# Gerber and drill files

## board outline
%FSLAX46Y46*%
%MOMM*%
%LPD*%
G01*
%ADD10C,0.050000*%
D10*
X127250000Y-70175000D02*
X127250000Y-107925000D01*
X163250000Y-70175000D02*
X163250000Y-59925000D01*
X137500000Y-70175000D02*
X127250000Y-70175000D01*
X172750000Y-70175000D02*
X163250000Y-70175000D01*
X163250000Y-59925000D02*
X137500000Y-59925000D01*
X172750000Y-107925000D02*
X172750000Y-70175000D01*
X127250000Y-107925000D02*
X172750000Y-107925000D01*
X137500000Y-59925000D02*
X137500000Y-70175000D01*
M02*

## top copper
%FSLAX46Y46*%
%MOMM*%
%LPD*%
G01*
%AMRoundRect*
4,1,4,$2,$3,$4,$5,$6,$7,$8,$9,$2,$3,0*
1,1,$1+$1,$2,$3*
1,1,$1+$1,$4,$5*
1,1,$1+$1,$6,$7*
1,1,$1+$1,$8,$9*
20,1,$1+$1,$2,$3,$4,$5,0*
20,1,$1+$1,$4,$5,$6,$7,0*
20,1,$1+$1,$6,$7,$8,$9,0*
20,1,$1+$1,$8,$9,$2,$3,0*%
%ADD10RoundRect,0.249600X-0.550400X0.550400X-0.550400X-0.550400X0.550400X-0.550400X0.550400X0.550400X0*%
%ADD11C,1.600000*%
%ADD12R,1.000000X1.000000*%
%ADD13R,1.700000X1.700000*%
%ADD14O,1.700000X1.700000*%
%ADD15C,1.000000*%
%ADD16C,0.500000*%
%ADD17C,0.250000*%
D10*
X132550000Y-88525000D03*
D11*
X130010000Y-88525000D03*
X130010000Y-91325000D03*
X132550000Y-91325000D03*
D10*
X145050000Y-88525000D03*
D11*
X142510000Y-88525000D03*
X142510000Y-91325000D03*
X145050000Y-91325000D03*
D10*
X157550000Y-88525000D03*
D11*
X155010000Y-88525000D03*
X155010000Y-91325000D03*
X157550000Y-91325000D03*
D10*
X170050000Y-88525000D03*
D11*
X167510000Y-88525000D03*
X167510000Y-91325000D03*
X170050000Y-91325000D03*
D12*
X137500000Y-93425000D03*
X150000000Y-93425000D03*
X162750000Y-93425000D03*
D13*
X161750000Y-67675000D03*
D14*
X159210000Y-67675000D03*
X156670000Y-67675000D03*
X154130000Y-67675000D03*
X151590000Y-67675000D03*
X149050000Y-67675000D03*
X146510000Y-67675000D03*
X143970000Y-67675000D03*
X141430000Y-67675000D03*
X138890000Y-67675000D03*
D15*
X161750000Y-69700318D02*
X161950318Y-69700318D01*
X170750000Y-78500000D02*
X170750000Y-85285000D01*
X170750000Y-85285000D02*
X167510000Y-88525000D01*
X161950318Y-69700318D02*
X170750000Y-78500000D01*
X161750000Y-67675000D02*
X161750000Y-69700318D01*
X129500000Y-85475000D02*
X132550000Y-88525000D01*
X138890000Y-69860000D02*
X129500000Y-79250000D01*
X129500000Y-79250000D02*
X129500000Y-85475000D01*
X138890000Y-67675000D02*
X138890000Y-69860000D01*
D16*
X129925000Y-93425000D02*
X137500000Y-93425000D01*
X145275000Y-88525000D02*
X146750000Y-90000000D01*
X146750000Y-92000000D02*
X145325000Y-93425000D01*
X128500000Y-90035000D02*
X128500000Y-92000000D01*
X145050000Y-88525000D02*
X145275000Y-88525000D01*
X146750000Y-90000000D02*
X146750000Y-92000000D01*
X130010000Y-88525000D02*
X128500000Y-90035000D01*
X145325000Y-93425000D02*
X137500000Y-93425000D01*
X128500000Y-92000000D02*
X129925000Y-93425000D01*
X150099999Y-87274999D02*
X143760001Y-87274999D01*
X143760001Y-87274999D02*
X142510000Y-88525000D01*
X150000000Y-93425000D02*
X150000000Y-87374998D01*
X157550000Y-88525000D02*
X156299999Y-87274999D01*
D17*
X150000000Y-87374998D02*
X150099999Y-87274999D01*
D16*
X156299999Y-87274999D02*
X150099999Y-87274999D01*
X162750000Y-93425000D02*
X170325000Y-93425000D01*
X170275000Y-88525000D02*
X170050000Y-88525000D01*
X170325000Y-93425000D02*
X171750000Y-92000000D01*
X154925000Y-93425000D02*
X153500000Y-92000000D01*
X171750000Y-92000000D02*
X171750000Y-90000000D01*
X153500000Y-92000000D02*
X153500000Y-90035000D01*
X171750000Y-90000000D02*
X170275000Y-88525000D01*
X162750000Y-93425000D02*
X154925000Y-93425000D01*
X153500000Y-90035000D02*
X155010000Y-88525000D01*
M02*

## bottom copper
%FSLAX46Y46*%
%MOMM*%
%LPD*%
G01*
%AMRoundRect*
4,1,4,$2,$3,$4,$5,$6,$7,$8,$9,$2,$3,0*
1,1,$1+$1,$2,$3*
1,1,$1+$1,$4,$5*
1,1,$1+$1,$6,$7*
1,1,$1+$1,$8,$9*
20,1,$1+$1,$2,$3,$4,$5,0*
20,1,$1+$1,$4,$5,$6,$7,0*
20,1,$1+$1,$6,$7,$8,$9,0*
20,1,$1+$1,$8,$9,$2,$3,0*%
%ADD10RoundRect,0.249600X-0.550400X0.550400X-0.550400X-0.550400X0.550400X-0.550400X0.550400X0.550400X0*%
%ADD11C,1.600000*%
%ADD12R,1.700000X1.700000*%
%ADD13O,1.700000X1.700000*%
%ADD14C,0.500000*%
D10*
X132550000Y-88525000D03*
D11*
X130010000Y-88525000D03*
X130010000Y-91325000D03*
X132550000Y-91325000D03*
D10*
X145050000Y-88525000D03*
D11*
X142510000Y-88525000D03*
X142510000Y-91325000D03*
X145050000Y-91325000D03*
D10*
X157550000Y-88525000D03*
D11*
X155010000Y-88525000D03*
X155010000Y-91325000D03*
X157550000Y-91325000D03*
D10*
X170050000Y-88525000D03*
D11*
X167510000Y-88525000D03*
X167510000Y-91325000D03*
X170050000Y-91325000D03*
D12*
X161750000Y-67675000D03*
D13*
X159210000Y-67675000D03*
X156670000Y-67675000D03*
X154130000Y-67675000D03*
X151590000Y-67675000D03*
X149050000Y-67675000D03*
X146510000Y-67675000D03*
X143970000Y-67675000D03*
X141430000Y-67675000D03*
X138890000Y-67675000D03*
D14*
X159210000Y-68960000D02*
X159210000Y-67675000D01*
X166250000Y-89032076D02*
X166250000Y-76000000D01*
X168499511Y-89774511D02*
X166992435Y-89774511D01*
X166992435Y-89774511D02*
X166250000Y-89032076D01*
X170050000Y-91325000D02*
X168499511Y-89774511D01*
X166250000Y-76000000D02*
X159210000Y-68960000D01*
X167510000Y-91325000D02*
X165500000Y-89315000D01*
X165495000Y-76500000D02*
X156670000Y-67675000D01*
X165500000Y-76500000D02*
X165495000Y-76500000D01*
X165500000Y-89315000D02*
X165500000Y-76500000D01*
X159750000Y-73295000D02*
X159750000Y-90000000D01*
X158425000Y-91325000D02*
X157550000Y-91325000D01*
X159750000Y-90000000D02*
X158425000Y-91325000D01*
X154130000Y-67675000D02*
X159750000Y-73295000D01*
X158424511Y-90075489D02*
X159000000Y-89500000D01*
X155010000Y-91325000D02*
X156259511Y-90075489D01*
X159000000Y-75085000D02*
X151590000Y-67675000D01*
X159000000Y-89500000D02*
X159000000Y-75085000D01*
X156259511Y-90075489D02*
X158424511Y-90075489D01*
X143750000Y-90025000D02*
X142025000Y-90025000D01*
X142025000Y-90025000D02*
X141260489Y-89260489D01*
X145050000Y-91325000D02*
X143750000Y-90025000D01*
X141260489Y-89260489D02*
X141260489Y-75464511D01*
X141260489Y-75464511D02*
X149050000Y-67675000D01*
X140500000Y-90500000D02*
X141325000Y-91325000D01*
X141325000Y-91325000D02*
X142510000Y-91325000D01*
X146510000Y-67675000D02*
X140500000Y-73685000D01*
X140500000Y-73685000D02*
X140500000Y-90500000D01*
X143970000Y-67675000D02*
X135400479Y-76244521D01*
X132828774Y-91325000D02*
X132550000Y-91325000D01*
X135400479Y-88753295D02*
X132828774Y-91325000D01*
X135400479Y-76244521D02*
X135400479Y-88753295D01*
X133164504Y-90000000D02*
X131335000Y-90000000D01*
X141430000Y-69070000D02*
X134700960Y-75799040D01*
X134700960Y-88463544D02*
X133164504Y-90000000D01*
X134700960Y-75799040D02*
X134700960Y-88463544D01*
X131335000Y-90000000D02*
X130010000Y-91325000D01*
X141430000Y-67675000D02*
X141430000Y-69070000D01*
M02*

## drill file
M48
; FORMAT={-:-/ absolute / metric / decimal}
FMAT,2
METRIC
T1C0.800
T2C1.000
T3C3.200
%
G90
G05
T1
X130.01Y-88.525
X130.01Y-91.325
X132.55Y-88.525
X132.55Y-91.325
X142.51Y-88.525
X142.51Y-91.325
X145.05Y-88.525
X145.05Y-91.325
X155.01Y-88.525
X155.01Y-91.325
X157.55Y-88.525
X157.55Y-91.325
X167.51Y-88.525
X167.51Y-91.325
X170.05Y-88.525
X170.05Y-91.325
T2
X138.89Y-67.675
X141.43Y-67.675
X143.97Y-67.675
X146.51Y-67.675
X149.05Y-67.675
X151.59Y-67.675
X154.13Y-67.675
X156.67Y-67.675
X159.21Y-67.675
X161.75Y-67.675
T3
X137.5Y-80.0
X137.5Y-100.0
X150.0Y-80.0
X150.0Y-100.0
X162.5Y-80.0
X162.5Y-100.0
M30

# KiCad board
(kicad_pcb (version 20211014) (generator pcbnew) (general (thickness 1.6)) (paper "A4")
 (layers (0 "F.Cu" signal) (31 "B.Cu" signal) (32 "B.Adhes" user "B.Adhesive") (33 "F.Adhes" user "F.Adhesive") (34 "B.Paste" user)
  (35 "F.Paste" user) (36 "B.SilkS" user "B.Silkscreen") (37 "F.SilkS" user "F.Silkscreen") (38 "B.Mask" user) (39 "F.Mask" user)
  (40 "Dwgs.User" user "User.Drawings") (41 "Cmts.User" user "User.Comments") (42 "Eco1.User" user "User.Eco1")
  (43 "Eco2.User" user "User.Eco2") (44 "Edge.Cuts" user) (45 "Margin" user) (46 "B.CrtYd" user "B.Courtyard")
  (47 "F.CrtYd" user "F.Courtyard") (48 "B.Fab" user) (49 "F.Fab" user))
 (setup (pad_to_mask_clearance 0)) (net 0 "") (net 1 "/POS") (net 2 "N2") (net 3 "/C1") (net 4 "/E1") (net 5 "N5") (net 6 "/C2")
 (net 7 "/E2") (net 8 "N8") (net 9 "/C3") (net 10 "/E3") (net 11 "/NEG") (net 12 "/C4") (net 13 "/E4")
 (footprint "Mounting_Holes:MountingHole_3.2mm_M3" (layer "F.Cu") (at 137.5 100)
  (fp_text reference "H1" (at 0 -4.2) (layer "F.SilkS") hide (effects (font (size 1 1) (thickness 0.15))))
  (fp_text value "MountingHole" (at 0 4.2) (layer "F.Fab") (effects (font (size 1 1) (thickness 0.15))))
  (pad "" np_thru_hole circle locked (at 0 0) (size 3.2 3.2) (drill 3.2) (layers *.Cu *.Mask)))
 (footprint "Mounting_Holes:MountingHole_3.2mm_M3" (layer "F.Cu") (at 137.5 80)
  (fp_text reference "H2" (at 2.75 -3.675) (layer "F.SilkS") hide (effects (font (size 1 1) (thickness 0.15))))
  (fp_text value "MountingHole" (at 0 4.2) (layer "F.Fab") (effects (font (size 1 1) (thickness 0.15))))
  (pad "" np_thru_hole circle locked (at 0 0) (size 3.2 3.2) (drill 3.2) (layers *.Cu *.Mask)))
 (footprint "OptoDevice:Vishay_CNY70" (layer "F.Cu") (at 132.55 88.525 -90)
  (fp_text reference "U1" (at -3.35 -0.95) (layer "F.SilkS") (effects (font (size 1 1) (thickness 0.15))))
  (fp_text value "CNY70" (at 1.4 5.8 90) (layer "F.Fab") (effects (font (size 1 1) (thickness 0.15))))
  (pad "1" thru_hole roundrect (at 0 0 270) (size 1.6 1.6) (drill 0.8) (layers *.Cu *.Mask) (roundrect_rratio 0.156) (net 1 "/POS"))
  (pad "2" thru_hole circle (at 0 2.54 270) (size 1.6 1.6) (drill 0.8) (layers *.Cu *.Mask) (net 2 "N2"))
  (pad "3" thru_hole circle (at 2.8 2.54 270) (size 1.6 1.6) (drill 0.8) (layers *.Cu *.Mask) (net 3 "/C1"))
  (pad "4" thru_hole circle (at 2.8 0 270) (size 1.6 1.6) (drill 0.8) (layers *.Cu *.Mask) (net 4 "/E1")))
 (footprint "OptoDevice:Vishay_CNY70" (layer "F.Cu") (at 145.05 88.525 -90)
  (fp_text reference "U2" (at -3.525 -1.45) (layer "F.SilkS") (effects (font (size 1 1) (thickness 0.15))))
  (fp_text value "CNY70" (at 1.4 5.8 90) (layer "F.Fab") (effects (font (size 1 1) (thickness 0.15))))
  (pad "1" thru_hole roundrect (at 0 0 270) (size 1.6 1.6) (drill 0.8) (layers *.Cu *.Mask) (roundrect_rratio 0.156) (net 2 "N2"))
  (pad "2" thru_hole circle (at 0 2.54 270) (size 1.6 1.6) (drill 0.8) (layers *.Cu *.Mask) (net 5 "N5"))
  (pad "3" thru_hole circle (at 2.8 2.54 270) (size 1.6 1.6) (drill 0.8) (layers *.Cu *.Mask) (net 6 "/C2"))
  (pad "4" thru_hole circle (at 2.8 0 270) (size 1.6 1.6) (drill 0.8) (layers *.Cu *.Mask) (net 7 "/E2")))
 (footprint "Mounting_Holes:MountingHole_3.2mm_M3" (layer "F.Cu") (at 150 100)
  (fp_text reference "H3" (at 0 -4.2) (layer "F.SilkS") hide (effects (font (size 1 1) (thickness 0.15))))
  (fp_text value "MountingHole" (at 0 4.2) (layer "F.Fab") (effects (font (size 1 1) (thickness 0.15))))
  (pad "" np_thru_hole circle locked (at 0 0) (size 3.2 3.2) (drill 3.2) (layers *.Cu *.Mask)))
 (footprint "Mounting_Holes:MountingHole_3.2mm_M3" (layer "F.Cu") (at 150 80)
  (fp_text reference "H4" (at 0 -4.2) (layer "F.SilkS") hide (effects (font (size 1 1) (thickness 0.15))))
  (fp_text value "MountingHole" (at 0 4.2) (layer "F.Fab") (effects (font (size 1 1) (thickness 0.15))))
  (pad "" np_thru_hole circle locked (at 0 0) (size 3.2 3.2) (drill 3.2) (layers *.Cu *.Mask)))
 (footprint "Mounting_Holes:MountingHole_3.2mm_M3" (layer "F.Cu") (at 162.5 100)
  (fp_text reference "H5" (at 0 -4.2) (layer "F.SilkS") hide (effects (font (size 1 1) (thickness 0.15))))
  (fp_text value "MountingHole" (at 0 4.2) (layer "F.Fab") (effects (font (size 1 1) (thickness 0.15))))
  (pad "" np_thru_hole circle locked (at 0 0) (size 3.2 3.2) (drill 3.2) (layers *.Cu *.Mask)))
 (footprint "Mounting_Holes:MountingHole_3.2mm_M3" (layer "F.Cu") (at 162.5 80)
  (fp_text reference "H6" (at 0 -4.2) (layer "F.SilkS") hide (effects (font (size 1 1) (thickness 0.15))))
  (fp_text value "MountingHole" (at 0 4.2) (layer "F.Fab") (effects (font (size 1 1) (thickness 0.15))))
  (pad "" np_thru_hole circle locked (at 0 0) (size 3.2 3.2) (drill 3.2) (layers *.Cu *.Mask)))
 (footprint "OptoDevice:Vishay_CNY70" (layer "F.Cu") (at 157.55 88.525 -90)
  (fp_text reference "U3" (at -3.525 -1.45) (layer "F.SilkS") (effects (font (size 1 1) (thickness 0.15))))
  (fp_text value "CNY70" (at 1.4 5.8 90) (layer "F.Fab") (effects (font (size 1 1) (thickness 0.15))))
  (pad "1" thru_hole roundrect (at 0 0 270) (size 1.6 1.6) (drill 0.8) (layers *.Cu *.Mask) (roundrect_rratio 0.156) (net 5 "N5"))
  (pad "2" thru_hole circle (at 0 2.54 270) (size 1.6 1.6) (drill 0.8) (layers *.Cu *.Mask) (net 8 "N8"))
  (pad "3" thru_hole circle (at 2.8 2.54 270) (size 1.6 1.6) (drill 0.8) (layers *.Cu *.Mask) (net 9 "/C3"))
  (pad "4" thru_hole circle (at 2.8 0 270) (size 1.6 1.6) (drill 0.8) (layers *.Cu *.Mask) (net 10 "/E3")))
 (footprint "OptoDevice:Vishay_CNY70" (layer "F.Cu") (at 170.05 88.525 -90)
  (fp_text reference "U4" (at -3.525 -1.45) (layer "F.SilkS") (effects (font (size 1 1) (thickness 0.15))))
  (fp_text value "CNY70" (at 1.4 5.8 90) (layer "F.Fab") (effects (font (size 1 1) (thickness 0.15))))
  (pad "1" thru_hole roundrect (at 0 0 270) (size 1.6 1.6) (drill 0.8) (layers *.Cu *.Mask) (roundrect_rratio 0.156) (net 8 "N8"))
  (pad "2" thru_hole circle (at 0 2.54 270) (size 1.6 1.6) (drill 0.8) (layers *.Cu *.Mask) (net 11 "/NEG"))
  (pad "3" thru_hole circle (at 2.8 2.54 270) (size 1.6 1.6) (drill 0.8) (layers *.Cu *.Mask) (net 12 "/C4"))
  (pad "4" thru_hole circle (at 2.8 0 270) (size 1.6 1.6) (drill 0.8) (layers *.Cu *.Mask) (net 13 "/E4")))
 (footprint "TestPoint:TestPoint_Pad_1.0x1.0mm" (layer "F.Cu") (at 137.5 93.425)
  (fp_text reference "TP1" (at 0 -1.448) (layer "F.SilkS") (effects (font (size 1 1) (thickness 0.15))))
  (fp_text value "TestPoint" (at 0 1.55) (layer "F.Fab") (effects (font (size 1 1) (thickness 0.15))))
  (pad "1" smd rect locked (at 0 0) (size 1 1) (layers "F.Cu" "F.Mask") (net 2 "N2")))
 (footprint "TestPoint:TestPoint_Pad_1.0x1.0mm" (layer "F.Cu") (at 150 93.425)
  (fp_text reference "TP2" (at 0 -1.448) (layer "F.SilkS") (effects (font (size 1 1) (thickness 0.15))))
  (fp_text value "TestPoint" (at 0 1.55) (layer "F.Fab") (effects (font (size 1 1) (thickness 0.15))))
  (pad "1" smd rect locked (at 0 0) (size 1 1) (layers "F.Cu" "F.Mask") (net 5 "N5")))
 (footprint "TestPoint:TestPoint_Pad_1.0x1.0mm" (layer "F.Cu") (at 162.75 93.425)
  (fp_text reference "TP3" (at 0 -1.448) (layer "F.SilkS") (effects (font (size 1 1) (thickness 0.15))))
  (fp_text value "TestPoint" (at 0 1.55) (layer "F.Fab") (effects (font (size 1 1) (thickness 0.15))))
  (pad "1" smd rect locked (at 0 0) (size 1 1) (layers "F.Cu" "F.Mask") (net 8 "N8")))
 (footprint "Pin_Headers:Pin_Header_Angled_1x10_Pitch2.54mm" (layer "B.Cu") (at 161.75 67.675 90)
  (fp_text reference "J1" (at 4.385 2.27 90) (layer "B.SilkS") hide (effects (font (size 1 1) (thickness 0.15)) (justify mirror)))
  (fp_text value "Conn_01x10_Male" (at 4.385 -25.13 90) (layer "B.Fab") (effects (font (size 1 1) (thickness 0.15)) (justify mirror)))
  (pad "1" thru_hole rect (at 0 0 90) (size 1.7 1.7) (drill 1) (layers *.Cu *.Mask) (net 11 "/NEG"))
  (pad "2" thru_hole oval (at 0 -2.54 90) (size 1.7 1.7) (drill 1) (layers *.Cu *.Mask) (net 13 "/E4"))
  (pad "3" thru_hole oval (at 0 -5.08 90) (size 1.7 1.7) (drill 1) (layers *.Cu *.Mask) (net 12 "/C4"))
  (pad "4" thru_hole oval (at 0 -7.62 90) (size 1.7 1.7) (drill 1) (layers *.Cu *.Mask) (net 10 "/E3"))
  (pad "5" thru_hole oval (at 0 -10.16 90) (size 1.7 1.7) (drill 1) (layers *.Cu *.Mask) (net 9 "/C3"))
  (pad "6" thru_hole oval (at 0 -12.7 90) (size 1.7 1.7) (drill 1) (layers *.Cu *.Mask) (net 7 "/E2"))
  (pad "7" thru_hole oval (at 0 -15.24 90) (size 1.7 1.7) (drill 1) (layers *.Cu *.Mask) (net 6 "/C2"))
  (pad "8" thru_hole oval (at 0 -17.78 90) (size 1.7 1.7) (drill 1) (layers *.Cu *.Mask) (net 4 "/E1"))
  (pad "9" thru_hole oval (at 0 -20.32 90) (size 1.7 1.7) (drill 1) (layers *.Cu *.Mask) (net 3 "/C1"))
  (pad "10" thru_hole oval (at 0 -22.86 90) (size 1.7 1.7) (drill 1) (layers *.Cu *.Mask) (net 1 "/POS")))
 (gr_line (start 127.25 70.175) (end 127.25 107.925) (layer "Edge.Cuts") (width 0.05))
 (gr_line (start 163.25 70.175) (end 163.25 59.925) (layer "Edge.Cuts") (width 0.05))
 (gr_line (start 137.5 70.175) (end 127.25 70.175) (layer "Edge.Cuts") (width 0.05))
 (gr_line (start 172.75 70.175) (end 163.25 70.175) (layer "Edge.Cuts") (width 0.05))
 (gr_line (start 163.25 59.925) (end 137.5 59.925) (layer "Edge.Cuts") (width 0.05))
 (gr_line (start 172.75 107.925) (end 172.75 70.175) (layer "Edge.Cuts") (width 0.05))
 (gr_line (start 127.25 107.925) (end 172.75 107.925) (layer "Edge.Cuts") (width 0.05))
 (gr_line (start 137.5 59.925) (end 137.5 70.175) (layer "Edge.Cuts") (width 0.05))
 (segment (start 161.75 69.700318) (end 161.950318 69.700318) (width 1) (layer "F.Cu") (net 11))
 (segment (start 170.75 78.5) (end 170.75 85.285) (width 1) (layer "F.Cu") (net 11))
 (segment (start 170.75 85.285) (end 167.51 88.525) (width 1) (layer "F.Cu") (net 11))
 (segment (start 161.950318 69.700318) (end 170.75 78.5) (width 1) (layer "F.Cu") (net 11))
 (segment (start 161.75 67.675) (end 161.75 69.700318) (width 1) (layer "F.Cu") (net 11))
 (segment (start 129.5 85.475) (end 132.55 88.525) (width 1) (layer "F.Cu") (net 1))
 (segment (start 138.89 69.86) (end 129.5 79.25) (width 1) (layer "F.Cu") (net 1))
 (segment (start 129.5 79.25) (end 129.5 85.475) (width 1) (layer "F.Cu") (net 1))
 (segment (start 138.89 67.675) (end 138.89 69.86) (width 1) (layer "F.Cu") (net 1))
 (segment (start 159.21 68.96) (end 159.21 67.675) (width 0.5) (layer "B.Cu") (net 13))
 (segment (start 166.25 89.032076) (end 166.25 76) (width 0.5) (layer "B.Cu") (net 13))
 (segment (start 168.499511 89.774511) (end 166.992435 89.774511) (width 0.5) (layer "B.Cu") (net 13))
 (segment (start 166.992435 89.774511) (end 166.25 89.032076) (width 0.5) (layer "B.Cu") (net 13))
 (segment (start 170.05 91.325) (end 168.499511 89.774511) (width 0.5) (layer "B.Cu") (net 13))
 (segment (start 166.25 76) (end 159.21 68.96) (width 0.5) (layer "B.Cu") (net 13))
 (segment (start 167.51 91.325) (end 165.5 89.315) (width 0.5) (layer "B.Cu") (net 12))
 (segment (start 165.495 76.5) (end 156.67 67.675) (width 0.5) (layer "B.Cu") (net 12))
 (segment (start 165.5 76.5) (end 165.495 76.5) (width 0.5) (layer "B.Cu") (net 12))
 (segment (start 165.5 89.315) (end 165.5 76.5) (width 0.5) (layer "B.Cu") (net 12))
 (segment (start 159.75 73.295) (end 159.75 90) (width 0.5) (layer "B.Cu") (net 10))
 (segment (start 158.425 91.325) (end 157.55 91.325) (width 0.5) (layer "B.Cu") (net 10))
 (segment (start 159.75 90) (end 158.425 91.325) (width 0.5) (layer "B.Cu") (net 10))
 (segment (start 154.13 67.675) (end 159.75 73.295) (width 0.5) (layer "B.Cu") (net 10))
 (segment (start 158.424511 90.075489) (end 159 89.5) (width 0.5) (layer "B.Cu") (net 9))
 (segment (start 155.01 91.325) (end 156.259511 90.075489) (width 0.5) (layer "B.Cu") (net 9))
 (segment (start 159 75.085) (end 151.59 67.675) (width 0.5) (layer "B.Cu") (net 9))
 (segment (start 159 89.5) (end 159 75.085) (width 0.5) (layer "B.Cu") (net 9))
 (segment (start 156.259511 90.075489) (end 158.424511 90.075489) (width 0.5) (layer "B.Cu") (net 9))
 (segment (start 143.75 90.025) (end 142.025 90.025) (width 0.5) (layer "B.Cu") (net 7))
 (segment (start 142.025 90.025) (end 141.260489 89.260489) (width 0.5) (layer "B.Cu") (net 7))
 (segment (start 145.05 91.325) (end 143.75 90.025) (width 0.5) (layer "B.Cu") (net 7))
 (segment (start 141.260489 89.260489) (end 141.260489 75.464511) (width 0.5) (layer "B.Cu") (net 7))
 (segment (start 141.260489 75.464511) (end 149.05 67.675) (width 0.5) (layer "B.Cu") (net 7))
 (segment (start 140.5 90.5) (end 141.325 91.325) (width 0.5) (layer "B.Cu") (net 6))
 (segment (start 141.325 91.325) (end 142.51 91.325) (width 0.5) (layer "B.Cu") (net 6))
 (segment (start 146.51 67.675) (end 140.5 73.685) (width 0.5) (layer "B.Cu") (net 6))
 (segment (start 140.5 73.685) (end 140.5 90.5) (width 0.5) (layer "B.Cu") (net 6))
 (segment (start 143.97 67.675) (end 135.400479 76.244521) (width 0.5) (layer "B.Cu") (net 4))
 (segment (start 132.828774 91.325) (end 132.55 91.325) (width 0.5) (layer "B.Cu") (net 4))
 (segment (start 135.400479 88.753295) (end 132.828774 91.325) (width 0.5) (layer "B.Cu") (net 4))
 (segment (start 135.400479 76.244521) (end 135.400479 88.753295) (width 0.5) (layer "B.Cu") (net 4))
 (segment (start 133.164504 90) (end 131.335 90) (width 0.5) (layer "B.Cu") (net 3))
 (segment (start 141.43 69.07) (end 134.70096 75.79904) (width 0.5) (layer "B.Cu") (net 3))
 (segment (start 134.70096 88.463544) (end 133.164504 90) (width 0.5) (layer "B.Cu") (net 3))
 (segment (start 134.70096 75.79904) (end 134.70096 88.463544) (width 0.5) (layer "B.Cu") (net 3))
 (segment (start 131.335 90) (end 130.01 91.325) (width 0.5) (layer "B.Cu") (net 3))
 (segment (start 141.43 67.675) (end 141.43 69.07) (width 0.5) (layer "B.Cu") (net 3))
 (segment (start 129.925 93.425) (end 137.5 93.425) (width 0.5) (layer "F.Cu") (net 2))
 (segment (start 145.275 88.525) (end 146.75 90) (width 0.5) (layer "F.Cu") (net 2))
 (segment (start 146.75 92) (end 145.325 93.425) (width 0.5) (layer "F.Cu") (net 2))
 (segment (start 128.5 90.035) (end 128.5 92) (width 0.5) (layer "F.Cu") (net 2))
 (segment (start 145.05 88.525) (end 145.275 88.525) (width 0.5) (layer "F.Cu") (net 2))
 (segment (start 146.75 90) (end 146.75 92) (width 0.5) (layer "F.Cu") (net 2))
 (segment (start 130.01 88.525) (end 128.5 90.035) (width 0.5) (layer "F.Cu") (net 2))
 (segment (start 145.325 93.425) (end 137.5 93.425) (width 0.5) (layer "F.Cu") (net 2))
 (segment (start 128.5 92) (end 129.925 93.425) (width 0.5) (layer "F.Cu") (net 2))
 (segment (start 150.099999 87.274999) (end 143.760001 87.274999) (width 0.5) (layer "F.Cu") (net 5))
 (segment (start 143.760001 87.274999) (end 142.51 88.525) (width 0.5) (layer "F.Cu") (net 5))
 (segment (start 150 93.425) (end 150 87.374998) (width 0.5) (layer "F.Cu") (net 5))
 (segment (start 157.55 88.525) (end 156.299999 87.274999) (width 0.5) (layer "F.Cu") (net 5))
 (segment (start 150 87.374998) (end 150.099999 87.274999) (width 0.25) (layer "F.Cu") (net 5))
 (segment (start 156.299999 87.274999) (end 150.099999 87.274999) (width 0.5) (layer "F.Cu") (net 5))
 (segment (start 162.75 93.425) (end 170.325 93.425) (width 0.5) (layer "F.Cu") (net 8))
 (segment (start 170.275 88.525) (end 170.05 88.525) (width 0.5) (layer "F.Cu") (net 8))
 (segment (start 170.325 93.425) (end 171.75 92) (width 0.5) (layer "F.Cu") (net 8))
 (segment (start 154.925 93.425) (end 153.5 92) (width 0.5) (layer "F.Cu") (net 8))
 (segment (start 171.75 92) (end 171.75 90) (width 0.5) (layer "F.Cu") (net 8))
 (segment (start 153.5 92) (end 153.5 90.035) (width 0.5) (layer "F.Cu") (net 8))
 (segment (start 171.75 90) (end 170.275 88.525) (width 0.5) (layer "F.Cu") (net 8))
 (segment (start 162.75 93.425) (end 154.925 93.425) (width 0.5) (layer "F.Cu") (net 8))
 (segment (start 153.5 90.035) (end 155.01 88.525) (width 0.5) (layer "F.Cu") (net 8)))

